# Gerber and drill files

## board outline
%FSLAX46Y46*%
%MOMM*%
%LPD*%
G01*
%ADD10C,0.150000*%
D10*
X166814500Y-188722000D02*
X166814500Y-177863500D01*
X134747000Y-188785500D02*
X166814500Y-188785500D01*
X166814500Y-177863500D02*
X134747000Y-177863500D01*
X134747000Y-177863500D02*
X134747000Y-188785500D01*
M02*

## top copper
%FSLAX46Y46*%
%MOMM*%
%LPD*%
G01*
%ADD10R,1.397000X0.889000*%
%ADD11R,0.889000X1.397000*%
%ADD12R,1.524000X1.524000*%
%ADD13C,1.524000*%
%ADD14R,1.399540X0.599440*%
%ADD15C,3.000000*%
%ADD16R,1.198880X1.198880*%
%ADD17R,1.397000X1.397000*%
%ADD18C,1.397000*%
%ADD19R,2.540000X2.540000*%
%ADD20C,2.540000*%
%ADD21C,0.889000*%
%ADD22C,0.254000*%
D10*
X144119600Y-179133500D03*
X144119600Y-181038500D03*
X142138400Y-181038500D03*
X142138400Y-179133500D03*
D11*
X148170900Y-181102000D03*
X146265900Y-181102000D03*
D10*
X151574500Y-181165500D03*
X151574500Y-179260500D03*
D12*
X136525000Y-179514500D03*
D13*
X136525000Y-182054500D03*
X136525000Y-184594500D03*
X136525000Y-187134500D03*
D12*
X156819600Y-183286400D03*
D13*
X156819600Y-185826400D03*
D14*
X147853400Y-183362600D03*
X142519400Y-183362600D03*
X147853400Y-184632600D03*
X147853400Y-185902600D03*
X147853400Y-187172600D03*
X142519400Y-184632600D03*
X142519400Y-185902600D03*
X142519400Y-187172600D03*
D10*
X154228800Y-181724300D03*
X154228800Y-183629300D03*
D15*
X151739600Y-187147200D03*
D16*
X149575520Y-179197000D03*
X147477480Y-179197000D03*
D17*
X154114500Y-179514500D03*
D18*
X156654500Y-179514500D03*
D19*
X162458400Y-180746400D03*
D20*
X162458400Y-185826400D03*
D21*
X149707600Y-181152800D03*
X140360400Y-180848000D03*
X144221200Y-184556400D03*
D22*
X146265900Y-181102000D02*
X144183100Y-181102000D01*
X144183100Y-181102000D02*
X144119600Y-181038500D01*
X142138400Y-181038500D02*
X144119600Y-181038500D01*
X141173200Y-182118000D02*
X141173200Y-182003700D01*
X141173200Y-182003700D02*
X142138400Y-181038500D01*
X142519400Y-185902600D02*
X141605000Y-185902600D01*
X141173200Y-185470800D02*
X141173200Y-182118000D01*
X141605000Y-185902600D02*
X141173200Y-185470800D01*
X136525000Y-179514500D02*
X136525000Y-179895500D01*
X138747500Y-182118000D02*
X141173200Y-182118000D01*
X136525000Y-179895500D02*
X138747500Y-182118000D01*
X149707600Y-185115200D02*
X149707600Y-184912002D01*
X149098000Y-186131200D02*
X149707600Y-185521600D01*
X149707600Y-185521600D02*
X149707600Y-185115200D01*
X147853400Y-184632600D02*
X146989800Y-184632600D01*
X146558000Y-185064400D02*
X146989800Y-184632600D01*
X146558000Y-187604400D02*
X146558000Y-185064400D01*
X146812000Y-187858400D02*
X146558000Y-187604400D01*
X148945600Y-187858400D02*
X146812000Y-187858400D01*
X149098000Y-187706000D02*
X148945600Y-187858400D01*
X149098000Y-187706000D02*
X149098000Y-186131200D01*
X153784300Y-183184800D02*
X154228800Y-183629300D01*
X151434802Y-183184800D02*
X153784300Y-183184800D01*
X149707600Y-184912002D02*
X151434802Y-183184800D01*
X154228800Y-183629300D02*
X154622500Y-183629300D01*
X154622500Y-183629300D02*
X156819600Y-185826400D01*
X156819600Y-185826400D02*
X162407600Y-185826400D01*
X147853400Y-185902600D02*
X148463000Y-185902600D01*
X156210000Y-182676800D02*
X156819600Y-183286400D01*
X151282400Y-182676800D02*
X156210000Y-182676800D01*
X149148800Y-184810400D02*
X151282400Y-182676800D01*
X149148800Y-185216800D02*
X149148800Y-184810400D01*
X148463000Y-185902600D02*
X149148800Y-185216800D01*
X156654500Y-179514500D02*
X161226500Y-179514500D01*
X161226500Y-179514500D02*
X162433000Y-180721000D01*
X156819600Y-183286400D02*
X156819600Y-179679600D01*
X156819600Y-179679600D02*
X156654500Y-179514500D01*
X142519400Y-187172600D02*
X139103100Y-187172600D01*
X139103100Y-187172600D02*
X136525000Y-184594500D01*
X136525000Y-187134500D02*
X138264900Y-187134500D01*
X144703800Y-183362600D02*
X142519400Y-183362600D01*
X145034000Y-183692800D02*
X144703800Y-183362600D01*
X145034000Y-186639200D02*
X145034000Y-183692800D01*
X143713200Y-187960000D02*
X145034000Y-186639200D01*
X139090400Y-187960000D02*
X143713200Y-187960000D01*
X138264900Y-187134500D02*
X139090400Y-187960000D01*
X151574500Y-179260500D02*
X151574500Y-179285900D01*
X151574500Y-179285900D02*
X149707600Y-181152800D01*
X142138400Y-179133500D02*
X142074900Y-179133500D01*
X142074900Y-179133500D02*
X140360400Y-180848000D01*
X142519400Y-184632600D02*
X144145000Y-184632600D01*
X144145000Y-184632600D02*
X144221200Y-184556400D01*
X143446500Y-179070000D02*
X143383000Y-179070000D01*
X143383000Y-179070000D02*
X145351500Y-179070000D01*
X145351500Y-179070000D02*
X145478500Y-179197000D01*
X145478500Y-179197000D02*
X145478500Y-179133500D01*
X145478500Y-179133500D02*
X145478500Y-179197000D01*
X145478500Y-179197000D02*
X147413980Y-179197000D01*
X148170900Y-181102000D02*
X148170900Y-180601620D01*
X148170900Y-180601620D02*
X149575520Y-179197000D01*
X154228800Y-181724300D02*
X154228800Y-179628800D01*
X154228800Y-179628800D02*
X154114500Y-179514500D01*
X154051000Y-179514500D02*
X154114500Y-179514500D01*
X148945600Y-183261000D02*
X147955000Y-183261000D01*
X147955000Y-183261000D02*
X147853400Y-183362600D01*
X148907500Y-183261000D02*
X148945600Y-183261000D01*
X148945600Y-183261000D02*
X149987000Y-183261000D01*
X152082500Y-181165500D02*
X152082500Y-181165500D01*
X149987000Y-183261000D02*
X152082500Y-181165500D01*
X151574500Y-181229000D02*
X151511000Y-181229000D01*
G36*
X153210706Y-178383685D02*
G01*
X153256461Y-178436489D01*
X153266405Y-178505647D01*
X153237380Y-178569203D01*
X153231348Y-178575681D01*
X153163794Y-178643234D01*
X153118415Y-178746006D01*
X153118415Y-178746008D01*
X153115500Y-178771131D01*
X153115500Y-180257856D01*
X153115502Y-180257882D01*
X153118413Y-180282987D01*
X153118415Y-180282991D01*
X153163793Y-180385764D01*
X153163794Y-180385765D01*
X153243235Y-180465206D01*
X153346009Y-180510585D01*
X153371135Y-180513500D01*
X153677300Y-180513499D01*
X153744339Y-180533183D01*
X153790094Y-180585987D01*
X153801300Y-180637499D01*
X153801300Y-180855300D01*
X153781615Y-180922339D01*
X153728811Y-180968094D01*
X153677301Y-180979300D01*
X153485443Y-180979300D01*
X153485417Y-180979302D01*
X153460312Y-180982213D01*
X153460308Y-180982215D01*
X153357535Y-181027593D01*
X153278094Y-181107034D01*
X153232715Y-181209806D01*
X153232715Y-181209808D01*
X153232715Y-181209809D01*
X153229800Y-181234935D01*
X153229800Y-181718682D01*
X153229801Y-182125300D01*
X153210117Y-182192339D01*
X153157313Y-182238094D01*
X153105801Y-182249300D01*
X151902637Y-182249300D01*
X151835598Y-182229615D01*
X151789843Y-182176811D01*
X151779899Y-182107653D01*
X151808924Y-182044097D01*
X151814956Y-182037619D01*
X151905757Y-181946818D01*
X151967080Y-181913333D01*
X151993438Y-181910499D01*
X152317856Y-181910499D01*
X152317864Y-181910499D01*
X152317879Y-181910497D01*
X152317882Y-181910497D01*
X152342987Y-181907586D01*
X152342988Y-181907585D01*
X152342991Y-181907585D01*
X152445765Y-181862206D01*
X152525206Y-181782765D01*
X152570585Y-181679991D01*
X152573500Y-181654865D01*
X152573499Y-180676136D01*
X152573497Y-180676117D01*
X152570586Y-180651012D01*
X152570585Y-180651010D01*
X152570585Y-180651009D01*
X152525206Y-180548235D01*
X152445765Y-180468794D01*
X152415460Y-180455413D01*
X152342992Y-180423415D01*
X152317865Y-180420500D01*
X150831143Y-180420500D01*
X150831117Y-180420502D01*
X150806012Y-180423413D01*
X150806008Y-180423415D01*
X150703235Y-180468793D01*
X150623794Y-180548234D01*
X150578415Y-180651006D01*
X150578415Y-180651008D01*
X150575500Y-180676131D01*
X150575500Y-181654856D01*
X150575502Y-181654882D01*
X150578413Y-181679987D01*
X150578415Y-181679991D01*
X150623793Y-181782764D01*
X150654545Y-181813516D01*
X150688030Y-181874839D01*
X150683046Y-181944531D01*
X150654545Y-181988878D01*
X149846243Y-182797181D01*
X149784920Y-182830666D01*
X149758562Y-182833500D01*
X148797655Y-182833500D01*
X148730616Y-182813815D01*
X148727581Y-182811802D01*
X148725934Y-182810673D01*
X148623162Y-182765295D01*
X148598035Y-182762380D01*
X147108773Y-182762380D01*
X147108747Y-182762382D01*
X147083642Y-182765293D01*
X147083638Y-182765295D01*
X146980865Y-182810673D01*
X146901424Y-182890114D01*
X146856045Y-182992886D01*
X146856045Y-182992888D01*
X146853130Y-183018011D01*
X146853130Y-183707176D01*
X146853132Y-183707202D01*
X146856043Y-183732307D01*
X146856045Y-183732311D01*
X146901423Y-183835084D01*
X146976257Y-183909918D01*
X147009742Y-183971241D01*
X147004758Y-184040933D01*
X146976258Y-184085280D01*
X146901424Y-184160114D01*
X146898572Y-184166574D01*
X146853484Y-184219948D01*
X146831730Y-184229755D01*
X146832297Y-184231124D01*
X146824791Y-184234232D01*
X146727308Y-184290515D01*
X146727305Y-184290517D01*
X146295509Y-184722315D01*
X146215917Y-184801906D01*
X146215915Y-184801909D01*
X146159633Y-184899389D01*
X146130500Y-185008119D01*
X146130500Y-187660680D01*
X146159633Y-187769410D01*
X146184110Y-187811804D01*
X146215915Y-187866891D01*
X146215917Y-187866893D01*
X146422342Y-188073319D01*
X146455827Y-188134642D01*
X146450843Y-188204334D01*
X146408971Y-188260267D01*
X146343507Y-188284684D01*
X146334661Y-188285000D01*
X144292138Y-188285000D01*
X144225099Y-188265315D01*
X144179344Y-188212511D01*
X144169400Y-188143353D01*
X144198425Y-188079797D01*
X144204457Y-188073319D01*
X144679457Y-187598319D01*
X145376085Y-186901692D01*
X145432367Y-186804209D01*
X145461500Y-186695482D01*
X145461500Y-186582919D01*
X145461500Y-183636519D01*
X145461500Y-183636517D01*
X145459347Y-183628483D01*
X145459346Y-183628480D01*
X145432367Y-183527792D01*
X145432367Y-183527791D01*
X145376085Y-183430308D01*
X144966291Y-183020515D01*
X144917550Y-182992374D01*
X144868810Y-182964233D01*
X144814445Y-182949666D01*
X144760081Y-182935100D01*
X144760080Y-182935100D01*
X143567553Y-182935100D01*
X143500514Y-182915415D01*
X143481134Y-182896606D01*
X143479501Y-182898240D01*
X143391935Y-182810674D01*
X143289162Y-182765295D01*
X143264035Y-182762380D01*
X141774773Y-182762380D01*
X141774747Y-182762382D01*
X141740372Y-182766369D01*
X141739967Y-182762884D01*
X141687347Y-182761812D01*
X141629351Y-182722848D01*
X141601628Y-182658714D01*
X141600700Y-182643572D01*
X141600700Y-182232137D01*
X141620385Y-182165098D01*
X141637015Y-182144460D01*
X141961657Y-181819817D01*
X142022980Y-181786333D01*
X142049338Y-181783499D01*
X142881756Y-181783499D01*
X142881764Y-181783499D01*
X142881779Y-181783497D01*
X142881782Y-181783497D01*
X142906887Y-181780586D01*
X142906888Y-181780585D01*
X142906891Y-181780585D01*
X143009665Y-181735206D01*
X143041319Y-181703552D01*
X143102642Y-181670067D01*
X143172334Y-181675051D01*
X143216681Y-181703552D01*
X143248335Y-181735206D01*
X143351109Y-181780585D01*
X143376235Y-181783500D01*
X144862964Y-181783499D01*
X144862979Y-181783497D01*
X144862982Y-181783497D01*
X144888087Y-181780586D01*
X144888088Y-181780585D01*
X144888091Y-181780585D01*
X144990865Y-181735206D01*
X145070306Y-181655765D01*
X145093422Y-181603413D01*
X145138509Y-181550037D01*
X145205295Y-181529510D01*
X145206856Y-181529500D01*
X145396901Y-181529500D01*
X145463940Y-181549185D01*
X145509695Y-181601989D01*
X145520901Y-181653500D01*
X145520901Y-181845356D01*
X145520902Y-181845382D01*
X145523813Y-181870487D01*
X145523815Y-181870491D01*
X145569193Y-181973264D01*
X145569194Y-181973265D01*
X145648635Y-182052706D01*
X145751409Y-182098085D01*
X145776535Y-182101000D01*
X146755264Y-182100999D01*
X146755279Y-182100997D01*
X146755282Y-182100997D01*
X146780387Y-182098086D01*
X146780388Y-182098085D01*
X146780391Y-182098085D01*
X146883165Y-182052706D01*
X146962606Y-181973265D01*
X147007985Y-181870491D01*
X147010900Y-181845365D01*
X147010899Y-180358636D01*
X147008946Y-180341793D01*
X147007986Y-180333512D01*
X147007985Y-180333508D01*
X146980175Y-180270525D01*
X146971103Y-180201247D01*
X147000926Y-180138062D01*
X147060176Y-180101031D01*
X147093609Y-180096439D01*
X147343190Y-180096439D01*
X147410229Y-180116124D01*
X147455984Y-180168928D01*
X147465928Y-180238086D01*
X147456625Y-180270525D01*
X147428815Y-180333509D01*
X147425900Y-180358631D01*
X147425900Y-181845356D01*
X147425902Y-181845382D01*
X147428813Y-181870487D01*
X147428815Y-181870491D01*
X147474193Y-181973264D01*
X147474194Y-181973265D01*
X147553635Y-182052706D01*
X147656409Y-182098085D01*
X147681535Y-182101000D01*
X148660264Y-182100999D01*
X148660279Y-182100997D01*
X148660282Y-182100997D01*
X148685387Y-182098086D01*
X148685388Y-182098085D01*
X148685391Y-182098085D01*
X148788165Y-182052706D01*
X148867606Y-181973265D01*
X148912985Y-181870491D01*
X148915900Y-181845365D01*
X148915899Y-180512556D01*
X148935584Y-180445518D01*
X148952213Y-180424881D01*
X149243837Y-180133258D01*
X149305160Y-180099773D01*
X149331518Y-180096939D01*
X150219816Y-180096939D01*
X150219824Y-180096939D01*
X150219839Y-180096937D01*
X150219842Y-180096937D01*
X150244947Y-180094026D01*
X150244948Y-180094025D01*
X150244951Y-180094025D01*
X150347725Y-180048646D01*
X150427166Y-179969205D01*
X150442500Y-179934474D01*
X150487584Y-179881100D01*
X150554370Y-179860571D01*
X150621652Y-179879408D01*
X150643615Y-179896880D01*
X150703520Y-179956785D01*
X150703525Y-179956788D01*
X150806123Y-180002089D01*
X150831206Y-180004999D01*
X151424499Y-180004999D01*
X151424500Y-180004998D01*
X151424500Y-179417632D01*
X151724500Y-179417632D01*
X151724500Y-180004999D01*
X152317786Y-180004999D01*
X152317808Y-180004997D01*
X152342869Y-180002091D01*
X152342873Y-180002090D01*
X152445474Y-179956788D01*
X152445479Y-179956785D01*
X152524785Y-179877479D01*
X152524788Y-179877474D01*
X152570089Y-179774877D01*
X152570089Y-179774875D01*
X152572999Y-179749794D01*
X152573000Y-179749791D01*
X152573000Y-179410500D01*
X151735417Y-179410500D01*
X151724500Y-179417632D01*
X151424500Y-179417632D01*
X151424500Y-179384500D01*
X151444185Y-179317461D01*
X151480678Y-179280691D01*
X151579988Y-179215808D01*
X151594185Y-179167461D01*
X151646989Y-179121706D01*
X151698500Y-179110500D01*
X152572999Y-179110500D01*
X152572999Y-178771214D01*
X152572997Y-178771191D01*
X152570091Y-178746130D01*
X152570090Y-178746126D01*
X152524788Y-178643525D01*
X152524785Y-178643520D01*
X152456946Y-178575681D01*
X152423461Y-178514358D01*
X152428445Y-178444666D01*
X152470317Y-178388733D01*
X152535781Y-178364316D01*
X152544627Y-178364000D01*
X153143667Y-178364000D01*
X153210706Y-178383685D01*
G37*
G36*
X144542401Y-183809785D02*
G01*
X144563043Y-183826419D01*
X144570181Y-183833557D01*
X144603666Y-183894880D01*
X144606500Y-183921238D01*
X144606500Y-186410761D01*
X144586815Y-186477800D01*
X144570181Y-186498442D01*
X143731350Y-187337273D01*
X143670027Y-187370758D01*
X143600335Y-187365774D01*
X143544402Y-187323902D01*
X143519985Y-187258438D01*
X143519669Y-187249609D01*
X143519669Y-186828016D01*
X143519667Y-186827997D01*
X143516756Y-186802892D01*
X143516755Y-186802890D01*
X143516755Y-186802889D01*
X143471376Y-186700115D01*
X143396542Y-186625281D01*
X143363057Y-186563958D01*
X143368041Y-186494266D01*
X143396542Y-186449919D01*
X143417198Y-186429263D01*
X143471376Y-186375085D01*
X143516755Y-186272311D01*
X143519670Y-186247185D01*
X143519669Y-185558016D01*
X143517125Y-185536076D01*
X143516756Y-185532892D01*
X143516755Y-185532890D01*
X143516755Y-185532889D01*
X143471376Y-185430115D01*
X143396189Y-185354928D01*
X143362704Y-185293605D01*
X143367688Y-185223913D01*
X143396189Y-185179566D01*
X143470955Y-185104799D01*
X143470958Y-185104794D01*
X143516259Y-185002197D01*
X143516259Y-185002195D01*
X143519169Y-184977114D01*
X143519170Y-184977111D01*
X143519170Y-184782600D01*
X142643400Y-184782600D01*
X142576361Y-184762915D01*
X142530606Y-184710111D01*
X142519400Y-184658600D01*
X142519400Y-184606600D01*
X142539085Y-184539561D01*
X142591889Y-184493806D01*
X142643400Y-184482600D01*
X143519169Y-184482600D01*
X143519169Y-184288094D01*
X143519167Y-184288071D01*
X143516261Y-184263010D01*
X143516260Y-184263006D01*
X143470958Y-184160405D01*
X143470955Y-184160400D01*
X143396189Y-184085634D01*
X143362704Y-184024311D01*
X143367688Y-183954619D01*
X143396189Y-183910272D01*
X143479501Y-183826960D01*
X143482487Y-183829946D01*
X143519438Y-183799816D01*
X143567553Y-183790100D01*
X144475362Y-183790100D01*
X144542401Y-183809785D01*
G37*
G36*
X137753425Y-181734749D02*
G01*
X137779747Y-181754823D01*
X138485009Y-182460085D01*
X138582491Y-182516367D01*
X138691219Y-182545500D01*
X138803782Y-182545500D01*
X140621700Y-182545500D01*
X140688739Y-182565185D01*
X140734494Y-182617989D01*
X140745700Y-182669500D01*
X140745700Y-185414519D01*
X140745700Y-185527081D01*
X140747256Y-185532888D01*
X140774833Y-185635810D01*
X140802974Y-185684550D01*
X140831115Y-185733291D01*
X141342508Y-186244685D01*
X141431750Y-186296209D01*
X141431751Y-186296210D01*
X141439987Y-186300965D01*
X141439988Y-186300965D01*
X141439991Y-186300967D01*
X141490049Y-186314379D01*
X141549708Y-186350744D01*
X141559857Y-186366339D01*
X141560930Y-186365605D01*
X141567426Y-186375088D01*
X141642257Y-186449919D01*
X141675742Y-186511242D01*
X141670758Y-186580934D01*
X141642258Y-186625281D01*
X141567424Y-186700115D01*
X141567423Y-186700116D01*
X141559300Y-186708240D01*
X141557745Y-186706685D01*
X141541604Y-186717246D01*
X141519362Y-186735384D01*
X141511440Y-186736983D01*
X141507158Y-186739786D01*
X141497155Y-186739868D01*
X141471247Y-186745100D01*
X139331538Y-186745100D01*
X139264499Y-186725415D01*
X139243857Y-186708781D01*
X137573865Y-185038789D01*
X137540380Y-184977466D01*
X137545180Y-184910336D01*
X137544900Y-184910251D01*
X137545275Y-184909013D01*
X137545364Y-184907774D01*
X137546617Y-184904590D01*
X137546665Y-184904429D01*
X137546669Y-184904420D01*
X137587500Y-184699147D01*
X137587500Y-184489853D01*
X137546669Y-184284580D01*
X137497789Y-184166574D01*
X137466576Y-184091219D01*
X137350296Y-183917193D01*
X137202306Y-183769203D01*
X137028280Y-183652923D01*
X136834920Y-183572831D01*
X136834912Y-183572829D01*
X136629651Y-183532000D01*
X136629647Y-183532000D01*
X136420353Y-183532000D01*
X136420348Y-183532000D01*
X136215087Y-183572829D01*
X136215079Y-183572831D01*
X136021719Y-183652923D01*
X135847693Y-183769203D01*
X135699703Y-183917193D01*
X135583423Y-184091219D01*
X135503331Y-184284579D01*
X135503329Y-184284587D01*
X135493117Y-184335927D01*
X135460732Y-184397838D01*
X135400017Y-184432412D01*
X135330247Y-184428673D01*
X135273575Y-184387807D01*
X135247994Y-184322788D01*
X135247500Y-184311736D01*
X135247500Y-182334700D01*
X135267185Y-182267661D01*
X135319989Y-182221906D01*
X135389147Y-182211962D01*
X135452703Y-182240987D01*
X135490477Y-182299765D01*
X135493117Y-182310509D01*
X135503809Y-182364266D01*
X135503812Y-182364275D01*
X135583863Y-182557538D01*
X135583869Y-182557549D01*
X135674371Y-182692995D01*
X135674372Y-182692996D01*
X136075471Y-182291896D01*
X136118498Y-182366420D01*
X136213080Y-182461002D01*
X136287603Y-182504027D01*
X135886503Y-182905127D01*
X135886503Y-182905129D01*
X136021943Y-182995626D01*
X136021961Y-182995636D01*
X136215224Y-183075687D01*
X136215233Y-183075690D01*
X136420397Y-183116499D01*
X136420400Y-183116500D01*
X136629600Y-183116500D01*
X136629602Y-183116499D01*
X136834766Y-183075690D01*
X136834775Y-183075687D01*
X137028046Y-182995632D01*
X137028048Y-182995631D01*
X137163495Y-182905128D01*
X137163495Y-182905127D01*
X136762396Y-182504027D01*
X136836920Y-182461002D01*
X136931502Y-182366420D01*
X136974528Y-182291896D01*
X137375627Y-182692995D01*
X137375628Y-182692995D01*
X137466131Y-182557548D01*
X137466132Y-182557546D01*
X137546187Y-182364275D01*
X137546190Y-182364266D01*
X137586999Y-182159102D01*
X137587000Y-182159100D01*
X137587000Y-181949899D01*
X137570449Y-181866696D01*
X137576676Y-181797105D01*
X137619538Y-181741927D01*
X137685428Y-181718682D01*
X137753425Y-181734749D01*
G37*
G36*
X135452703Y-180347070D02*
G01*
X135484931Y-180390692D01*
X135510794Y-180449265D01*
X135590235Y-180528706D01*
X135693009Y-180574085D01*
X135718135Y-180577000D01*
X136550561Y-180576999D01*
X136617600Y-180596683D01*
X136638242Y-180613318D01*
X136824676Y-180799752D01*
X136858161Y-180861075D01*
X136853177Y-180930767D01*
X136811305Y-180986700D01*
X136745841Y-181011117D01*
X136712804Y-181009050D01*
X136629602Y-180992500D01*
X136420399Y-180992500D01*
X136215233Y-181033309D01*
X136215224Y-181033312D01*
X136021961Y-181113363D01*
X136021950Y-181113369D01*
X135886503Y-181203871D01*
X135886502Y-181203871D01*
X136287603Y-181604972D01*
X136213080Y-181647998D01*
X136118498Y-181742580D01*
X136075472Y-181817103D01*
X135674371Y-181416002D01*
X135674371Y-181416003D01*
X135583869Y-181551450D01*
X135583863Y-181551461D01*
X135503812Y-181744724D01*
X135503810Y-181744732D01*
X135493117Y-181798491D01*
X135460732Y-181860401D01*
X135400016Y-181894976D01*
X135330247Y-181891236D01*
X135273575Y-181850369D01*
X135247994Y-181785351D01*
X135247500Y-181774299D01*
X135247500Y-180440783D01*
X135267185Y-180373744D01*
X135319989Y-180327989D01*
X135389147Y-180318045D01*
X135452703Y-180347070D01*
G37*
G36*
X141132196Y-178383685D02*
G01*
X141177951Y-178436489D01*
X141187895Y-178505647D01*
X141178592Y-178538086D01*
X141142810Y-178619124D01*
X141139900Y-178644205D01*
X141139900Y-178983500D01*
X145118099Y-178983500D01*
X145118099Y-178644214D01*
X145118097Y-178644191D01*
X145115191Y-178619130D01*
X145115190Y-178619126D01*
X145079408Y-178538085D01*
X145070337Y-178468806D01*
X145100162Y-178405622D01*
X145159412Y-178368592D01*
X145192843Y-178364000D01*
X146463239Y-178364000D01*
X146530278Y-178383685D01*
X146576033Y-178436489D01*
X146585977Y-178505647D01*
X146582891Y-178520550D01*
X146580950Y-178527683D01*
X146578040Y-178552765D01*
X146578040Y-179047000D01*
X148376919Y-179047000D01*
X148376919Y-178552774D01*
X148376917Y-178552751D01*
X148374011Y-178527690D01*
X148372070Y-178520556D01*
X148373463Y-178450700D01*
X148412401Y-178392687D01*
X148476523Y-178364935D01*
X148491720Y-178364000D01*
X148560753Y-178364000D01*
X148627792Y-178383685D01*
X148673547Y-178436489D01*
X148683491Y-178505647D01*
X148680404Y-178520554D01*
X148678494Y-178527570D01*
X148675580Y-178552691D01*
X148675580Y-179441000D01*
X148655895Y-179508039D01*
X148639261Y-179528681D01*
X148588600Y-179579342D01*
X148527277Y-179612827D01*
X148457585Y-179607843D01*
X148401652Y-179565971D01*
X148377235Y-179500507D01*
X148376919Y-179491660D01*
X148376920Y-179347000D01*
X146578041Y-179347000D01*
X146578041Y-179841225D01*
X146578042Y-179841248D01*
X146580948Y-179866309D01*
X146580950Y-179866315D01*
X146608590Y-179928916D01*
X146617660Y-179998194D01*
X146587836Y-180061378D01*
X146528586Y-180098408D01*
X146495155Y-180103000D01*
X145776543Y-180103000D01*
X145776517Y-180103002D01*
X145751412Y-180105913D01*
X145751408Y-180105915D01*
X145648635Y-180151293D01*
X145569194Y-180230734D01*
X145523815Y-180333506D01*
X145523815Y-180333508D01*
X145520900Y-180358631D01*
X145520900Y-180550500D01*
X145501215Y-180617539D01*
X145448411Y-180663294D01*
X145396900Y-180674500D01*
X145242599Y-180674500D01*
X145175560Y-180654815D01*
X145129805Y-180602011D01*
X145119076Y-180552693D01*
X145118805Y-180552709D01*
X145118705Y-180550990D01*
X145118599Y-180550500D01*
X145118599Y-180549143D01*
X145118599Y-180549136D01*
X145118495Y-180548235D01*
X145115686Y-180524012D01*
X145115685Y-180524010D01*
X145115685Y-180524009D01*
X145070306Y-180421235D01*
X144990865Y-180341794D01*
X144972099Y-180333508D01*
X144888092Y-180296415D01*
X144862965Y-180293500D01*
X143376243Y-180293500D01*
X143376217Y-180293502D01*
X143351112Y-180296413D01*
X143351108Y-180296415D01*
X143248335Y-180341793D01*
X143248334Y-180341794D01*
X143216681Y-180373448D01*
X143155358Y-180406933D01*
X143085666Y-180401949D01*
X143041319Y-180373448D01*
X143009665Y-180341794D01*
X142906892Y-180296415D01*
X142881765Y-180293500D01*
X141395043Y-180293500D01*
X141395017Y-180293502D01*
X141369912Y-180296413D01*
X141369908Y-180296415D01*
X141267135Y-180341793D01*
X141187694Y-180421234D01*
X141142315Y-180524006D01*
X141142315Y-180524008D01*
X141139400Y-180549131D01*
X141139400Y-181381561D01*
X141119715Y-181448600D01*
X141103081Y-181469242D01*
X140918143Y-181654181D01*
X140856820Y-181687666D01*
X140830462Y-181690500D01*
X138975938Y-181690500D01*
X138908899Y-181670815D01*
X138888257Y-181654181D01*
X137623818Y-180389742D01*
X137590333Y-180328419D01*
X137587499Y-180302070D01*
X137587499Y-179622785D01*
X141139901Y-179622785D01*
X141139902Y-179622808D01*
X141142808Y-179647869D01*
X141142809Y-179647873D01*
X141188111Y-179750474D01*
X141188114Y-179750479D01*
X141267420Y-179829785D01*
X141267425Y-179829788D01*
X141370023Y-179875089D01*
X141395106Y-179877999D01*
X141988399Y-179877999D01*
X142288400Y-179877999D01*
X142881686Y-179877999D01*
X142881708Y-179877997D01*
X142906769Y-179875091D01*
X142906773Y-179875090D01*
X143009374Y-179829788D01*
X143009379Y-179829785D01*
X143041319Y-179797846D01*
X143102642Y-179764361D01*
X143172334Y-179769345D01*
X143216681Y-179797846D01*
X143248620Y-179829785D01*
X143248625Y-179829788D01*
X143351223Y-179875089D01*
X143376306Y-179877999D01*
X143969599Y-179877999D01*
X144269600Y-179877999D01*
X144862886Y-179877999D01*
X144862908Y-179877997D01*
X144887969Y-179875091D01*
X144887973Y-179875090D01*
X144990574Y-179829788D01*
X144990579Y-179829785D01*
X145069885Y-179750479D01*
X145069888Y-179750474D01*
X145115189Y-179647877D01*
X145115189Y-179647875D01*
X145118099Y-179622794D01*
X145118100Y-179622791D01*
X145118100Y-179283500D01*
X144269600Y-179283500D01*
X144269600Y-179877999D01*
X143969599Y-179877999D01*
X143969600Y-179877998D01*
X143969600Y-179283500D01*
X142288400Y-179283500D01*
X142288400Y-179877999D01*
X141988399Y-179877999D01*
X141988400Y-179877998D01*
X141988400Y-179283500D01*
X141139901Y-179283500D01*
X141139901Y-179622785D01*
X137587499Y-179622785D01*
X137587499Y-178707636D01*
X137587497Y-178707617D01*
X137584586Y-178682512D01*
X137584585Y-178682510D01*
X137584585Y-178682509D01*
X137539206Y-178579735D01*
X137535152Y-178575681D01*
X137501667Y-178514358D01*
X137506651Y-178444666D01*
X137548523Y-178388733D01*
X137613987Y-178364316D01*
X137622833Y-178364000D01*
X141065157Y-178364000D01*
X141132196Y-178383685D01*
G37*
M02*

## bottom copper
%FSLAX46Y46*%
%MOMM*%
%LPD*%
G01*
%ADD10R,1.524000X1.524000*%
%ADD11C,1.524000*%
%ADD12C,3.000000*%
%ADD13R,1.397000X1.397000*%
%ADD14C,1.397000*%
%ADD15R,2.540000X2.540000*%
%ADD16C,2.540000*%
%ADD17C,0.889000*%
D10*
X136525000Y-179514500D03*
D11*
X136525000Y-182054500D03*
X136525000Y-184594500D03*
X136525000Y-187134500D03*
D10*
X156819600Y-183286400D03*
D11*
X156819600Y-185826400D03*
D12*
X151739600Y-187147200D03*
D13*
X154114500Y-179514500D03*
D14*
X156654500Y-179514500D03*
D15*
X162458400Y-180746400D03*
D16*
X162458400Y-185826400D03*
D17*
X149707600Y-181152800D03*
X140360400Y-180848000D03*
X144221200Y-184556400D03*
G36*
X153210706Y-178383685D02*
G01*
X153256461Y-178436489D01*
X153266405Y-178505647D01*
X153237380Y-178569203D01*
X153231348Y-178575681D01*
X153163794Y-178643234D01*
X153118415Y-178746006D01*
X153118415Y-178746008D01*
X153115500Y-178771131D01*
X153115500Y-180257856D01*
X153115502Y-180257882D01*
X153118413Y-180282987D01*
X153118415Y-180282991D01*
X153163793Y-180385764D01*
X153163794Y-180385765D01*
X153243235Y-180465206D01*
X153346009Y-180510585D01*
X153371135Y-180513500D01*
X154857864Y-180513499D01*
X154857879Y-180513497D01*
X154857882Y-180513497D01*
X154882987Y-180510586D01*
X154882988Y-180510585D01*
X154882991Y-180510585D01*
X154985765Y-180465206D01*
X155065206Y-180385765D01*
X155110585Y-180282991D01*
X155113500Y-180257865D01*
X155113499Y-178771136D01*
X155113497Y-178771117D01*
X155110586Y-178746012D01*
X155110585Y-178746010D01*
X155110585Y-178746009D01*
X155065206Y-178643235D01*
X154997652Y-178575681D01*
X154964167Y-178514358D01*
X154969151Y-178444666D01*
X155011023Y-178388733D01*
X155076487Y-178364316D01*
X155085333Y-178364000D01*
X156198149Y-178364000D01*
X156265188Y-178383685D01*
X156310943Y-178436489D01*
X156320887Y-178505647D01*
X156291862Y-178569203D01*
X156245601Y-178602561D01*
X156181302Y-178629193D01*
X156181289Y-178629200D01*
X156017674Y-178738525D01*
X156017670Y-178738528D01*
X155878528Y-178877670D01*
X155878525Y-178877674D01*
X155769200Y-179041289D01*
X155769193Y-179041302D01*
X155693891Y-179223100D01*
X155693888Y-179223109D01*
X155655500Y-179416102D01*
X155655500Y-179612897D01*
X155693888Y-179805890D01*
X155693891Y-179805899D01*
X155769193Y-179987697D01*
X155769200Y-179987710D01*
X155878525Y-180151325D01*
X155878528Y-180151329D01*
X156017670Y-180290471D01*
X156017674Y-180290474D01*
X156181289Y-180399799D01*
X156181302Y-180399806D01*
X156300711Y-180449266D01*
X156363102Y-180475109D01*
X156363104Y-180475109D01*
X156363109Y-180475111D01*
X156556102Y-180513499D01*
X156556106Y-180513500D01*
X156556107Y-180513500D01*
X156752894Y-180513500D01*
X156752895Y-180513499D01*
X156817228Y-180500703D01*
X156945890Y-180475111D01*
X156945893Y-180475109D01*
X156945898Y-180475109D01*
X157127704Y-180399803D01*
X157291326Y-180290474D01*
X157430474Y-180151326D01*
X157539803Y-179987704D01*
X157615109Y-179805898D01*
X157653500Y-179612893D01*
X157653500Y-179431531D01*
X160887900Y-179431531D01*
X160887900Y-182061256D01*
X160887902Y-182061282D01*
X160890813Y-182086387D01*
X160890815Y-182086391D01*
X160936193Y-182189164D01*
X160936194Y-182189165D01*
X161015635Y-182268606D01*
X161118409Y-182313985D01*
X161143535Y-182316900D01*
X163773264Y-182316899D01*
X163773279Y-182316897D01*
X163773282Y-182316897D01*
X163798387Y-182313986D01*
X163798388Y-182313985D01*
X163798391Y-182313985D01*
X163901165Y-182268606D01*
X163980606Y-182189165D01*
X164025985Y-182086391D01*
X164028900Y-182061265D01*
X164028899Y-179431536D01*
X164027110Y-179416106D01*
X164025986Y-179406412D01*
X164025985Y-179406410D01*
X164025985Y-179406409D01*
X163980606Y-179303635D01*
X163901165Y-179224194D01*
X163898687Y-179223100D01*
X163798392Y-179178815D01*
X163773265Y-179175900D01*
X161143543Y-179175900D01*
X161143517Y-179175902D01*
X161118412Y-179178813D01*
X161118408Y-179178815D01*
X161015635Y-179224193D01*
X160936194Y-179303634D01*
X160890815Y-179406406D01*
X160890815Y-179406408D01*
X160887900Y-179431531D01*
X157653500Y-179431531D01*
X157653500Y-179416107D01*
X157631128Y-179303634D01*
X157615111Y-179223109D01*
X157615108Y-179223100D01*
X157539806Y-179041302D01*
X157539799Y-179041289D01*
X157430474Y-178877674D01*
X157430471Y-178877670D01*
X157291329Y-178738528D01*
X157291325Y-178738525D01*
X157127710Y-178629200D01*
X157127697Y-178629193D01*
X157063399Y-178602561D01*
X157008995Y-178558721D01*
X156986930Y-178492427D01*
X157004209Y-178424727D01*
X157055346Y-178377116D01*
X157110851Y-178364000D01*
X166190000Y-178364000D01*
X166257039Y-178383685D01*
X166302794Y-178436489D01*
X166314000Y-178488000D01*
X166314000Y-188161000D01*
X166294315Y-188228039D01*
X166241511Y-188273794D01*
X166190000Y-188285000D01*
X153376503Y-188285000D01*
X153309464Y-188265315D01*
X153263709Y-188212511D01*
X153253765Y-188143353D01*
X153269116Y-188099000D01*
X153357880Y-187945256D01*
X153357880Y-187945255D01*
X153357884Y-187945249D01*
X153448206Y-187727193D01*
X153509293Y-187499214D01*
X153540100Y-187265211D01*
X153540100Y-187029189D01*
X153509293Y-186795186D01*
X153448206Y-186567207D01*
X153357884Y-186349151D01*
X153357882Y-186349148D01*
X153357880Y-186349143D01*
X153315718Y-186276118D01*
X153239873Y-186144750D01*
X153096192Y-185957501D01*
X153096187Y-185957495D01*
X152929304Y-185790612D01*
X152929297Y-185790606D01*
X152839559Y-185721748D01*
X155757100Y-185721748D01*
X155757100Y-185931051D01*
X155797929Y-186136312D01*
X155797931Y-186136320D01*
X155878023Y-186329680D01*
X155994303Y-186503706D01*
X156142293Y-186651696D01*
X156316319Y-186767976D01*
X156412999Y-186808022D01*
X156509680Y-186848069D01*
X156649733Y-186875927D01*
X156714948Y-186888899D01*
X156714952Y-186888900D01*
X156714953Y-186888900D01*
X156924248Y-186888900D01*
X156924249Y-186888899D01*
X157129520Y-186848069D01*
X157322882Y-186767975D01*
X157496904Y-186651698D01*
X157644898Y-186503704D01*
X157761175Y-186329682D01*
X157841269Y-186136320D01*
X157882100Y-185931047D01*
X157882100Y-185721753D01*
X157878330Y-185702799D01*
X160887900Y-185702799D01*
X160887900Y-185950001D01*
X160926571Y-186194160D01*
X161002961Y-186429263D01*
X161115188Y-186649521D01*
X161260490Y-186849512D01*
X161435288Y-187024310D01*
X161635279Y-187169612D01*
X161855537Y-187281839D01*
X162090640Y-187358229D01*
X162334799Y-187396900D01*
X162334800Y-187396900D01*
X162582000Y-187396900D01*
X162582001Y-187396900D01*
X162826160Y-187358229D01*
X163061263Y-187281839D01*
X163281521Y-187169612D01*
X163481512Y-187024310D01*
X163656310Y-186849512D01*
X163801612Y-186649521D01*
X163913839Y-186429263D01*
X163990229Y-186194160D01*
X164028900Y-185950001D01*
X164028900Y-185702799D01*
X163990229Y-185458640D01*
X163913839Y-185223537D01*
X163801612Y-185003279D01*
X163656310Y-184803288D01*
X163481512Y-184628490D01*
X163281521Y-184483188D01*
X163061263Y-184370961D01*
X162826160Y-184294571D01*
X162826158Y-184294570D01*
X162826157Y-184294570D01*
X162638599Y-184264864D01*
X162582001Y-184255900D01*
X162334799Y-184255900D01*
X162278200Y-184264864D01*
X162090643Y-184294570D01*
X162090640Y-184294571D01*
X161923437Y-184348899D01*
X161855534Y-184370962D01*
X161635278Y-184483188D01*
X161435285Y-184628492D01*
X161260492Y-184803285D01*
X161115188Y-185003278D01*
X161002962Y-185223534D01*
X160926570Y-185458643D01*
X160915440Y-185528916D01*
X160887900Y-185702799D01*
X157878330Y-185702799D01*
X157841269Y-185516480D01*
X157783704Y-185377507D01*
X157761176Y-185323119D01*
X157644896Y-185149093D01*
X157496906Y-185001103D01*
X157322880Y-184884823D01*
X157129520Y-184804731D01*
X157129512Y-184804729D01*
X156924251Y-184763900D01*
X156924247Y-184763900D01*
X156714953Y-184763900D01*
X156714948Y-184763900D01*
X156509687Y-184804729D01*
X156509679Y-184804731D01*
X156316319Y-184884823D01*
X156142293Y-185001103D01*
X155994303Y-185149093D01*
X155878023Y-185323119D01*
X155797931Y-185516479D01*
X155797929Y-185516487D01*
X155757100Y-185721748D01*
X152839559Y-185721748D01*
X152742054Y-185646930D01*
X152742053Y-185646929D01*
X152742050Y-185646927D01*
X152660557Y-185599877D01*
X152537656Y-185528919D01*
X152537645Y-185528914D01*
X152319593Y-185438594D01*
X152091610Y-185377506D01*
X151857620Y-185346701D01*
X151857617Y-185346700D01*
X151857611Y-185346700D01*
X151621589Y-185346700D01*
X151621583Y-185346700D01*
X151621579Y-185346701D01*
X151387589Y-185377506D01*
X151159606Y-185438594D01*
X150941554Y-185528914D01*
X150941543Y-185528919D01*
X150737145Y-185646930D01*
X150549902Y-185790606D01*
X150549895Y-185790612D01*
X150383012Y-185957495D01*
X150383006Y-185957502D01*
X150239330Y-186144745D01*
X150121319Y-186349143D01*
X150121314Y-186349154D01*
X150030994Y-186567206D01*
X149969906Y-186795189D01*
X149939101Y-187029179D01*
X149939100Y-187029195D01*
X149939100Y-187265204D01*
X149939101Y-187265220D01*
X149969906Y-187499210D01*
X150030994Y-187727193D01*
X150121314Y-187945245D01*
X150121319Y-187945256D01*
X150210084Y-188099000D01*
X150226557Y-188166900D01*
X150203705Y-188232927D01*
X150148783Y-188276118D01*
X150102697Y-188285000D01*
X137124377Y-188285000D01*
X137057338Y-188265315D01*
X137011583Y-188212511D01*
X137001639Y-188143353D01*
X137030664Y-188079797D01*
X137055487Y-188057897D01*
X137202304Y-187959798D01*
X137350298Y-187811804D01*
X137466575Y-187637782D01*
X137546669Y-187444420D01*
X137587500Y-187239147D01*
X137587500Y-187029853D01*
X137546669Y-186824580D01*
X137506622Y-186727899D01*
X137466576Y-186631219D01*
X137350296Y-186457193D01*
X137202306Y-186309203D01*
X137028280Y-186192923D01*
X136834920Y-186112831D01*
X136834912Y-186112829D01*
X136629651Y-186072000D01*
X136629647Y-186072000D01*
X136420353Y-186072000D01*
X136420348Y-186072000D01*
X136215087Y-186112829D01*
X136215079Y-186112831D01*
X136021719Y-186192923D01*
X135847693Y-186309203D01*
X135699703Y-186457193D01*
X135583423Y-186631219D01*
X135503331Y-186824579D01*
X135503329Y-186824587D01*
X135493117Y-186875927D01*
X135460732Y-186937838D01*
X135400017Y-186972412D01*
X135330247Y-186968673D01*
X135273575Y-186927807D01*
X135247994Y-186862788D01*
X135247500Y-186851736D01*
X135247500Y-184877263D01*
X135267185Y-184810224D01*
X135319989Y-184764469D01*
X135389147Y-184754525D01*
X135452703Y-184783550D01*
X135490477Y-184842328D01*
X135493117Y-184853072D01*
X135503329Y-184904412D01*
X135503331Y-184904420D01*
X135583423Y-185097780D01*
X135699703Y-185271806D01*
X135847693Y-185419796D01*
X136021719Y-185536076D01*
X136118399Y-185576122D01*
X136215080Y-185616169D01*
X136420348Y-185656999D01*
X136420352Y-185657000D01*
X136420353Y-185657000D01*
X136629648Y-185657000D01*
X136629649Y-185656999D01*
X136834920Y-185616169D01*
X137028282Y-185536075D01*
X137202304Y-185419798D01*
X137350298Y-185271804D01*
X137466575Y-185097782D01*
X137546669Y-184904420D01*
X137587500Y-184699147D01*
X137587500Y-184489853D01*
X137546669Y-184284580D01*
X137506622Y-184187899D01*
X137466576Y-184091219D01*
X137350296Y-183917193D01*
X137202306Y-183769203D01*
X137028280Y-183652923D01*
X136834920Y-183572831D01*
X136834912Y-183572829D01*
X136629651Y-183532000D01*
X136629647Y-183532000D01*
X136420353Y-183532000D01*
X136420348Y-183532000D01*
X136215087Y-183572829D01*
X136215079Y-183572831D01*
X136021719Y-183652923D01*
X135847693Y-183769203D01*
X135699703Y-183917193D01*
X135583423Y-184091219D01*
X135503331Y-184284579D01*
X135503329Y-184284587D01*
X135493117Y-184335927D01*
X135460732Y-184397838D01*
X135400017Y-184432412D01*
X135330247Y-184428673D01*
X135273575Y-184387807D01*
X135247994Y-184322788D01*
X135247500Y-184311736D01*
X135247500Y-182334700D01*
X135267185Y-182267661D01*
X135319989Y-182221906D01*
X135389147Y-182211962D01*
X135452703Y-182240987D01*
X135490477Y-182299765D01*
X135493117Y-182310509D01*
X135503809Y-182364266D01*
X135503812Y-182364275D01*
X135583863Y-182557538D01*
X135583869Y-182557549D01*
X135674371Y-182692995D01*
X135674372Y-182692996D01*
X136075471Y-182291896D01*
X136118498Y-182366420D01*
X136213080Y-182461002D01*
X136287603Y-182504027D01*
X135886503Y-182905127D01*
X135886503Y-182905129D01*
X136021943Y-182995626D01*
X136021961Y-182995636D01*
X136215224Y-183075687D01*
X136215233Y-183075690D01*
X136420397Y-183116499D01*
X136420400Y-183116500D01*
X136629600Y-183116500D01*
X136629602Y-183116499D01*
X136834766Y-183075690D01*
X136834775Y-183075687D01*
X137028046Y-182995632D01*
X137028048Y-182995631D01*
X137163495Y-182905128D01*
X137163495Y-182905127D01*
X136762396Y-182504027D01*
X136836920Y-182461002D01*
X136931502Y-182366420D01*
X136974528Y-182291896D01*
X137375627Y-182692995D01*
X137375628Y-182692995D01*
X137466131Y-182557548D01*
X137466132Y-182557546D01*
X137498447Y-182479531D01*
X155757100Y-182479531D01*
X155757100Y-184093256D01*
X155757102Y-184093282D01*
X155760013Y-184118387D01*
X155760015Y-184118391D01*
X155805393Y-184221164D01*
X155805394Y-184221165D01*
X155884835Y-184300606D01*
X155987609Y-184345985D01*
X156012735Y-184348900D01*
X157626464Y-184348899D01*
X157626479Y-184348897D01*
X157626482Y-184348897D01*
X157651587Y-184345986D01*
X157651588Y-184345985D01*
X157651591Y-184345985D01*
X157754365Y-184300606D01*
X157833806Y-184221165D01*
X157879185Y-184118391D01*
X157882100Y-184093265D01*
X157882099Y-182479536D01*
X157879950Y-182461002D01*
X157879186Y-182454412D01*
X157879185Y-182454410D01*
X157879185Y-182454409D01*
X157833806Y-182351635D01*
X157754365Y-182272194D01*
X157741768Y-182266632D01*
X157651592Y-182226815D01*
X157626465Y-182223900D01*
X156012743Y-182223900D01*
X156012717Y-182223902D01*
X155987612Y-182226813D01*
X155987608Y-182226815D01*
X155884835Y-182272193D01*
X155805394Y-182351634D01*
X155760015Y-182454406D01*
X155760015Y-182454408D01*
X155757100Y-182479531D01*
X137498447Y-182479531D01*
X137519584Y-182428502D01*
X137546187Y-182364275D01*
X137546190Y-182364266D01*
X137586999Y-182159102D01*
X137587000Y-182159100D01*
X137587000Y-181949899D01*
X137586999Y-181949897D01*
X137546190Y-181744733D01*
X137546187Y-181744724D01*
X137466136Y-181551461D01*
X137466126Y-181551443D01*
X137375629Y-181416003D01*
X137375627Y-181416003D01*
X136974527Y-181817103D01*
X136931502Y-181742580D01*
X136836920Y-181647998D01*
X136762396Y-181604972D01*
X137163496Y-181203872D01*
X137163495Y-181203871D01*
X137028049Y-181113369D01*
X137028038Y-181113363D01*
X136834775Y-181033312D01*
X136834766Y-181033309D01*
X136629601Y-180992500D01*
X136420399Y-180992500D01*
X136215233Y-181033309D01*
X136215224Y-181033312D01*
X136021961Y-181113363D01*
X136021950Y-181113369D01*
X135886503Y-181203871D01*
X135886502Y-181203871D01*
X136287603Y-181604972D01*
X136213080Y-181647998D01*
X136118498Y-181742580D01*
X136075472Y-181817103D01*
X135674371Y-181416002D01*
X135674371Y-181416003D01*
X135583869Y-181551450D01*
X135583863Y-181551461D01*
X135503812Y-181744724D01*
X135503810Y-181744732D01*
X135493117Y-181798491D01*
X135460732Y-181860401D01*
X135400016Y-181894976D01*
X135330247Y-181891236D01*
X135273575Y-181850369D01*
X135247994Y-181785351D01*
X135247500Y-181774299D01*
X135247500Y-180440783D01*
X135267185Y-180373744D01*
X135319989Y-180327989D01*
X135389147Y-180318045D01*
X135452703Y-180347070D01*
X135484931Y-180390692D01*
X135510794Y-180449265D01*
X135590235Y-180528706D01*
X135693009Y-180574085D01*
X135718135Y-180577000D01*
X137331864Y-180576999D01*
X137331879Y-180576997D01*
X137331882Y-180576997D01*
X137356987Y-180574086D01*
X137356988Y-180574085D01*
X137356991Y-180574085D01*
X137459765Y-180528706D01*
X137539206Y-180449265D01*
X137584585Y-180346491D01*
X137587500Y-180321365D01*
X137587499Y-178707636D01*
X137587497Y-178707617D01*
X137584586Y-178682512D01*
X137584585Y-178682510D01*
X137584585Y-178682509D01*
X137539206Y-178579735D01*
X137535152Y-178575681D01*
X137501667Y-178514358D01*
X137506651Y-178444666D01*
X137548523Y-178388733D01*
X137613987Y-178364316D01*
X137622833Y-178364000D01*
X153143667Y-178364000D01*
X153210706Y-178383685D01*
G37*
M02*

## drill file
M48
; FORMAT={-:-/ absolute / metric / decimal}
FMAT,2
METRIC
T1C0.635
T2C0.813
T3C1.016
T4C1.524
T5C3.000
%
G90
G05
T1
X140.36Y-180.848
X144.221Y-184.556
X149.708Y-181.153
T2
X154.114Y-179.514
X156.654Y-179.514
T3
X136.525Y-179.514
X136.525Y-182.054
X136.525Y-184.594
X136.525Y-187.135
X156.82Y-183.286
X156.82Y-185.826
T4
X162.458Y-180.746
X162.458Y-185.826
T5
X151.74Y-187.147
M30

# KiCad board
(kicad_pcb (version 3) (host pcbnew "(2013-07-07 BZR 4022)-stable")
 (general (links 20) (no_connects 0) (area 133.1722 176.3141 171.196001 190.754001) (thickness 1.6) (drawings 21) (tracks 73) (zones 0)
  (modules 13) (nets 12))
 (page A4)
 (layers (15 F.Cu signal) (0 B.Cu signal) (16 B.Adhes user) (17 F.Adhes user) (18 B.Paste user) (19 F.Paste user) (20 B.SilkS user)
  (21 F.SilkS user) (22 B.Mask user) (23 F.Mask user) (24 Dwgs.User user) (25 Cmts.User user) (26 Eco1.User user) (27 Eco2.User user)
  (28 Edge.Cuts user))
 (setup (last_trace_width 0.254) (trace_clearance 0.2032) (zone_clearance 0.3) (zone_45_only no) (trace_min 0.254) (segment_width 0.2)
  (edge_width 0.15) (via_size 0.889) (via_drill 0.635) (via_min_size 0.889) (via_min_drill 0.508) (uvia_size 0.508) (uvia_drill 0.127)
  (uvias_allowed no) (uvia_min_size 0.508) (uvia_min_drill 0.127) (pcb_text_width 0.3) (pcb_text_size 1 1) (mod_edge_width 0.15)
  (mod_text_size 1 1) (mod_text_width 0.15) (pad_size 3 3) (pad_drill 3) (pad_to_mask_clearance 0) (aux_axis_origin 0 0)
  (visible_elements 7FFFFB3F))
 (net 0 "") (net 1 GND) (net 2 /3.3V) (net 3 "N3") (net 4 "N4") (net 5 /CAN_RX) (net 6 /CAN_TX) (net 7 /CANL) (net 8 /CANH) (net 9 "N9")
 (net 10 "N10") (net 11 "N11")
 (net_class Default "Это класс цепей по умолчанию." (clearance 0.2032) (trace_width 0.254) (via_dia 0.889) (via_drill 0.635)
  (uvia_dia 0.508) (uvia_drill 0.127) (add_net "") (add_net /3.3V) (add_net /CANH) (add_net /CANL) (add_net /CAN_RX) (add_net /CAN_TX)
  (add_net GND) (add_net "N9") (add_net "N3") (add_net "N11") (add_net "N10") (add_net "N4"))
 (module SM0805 (layer F.Cu) (at 144.1196 180.086 270)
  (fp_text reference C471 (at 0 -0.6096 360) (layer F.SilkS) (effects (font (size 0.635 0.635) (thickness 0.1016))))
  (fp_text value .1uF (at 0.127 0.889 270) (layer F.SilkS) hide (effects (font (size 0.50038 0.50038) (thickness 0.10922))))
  (pad 1 smd rect (at -0.9525 0 270) (size 0.889 1.397) (layers F.Cu F.Paste F.Mask) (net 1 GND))
  (pad 2 smd rect (at 0.9525 0 270) (size 0.889 1.397) (layers F.Cu F.Paste F.Mask) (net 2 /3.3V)))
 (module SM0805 (layer F.Cu) (at 142.1384 180.086 90)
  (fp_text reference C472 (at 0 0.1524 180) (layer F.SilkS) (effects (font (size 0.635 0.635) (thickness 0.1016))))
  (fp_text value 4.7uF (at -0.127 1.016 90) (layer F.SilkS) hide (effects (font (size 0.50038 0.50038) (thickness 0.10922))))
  (pad 1 smd rect (at -0.9525 0 90) (size 0.889 1.397) (layers F.Cu F.Paste F.Mask) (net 2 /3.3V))
  (pad 2 smd rect (at 0.9525 0 90) (size 0.889 1.397) (layers F.Cu F.Paste F.Mask) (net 1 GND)))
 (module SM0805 (layer F.Cu) (at 147.2184 181.102 180)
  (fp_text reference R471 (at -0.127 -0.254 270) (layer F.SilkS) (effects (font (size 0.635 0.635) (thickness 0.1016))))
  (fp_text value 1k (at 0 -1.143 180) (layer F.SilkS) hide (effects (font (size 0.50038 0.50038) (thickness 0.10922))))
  (pad 1 smd rect (at -0.9525 0 180) (size 0.889 1.397) (layers F.Cu F.Paste F.Mask) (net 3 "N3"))
  (pad 2 smd rect (at 0.9525 0 180) (size 0.889 1.397) (layers F.Cu F.Paste F.Mask) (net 2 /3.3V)))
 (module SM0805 (layer F.Cu) (at 151.5745 180.213 90)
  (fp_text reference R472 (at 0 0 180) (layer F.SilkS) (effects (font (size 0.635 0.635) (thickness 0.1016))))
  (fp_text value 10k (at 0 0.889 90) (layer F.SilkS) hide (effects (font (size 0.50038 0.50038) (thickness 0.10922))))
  (pad 1 smd rect (at -0.9525 0 90) (size 0.889 1.397) (layers F.Cu F.Paste F.Mask) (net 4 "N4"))
  (pad 2 smd rect (at 0.9525 0 90) (size 0.889 1.397) (layers F.Cu F.Paste F.Mask) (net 1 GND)))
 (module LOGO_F (layer B.Cu) (at 146.4564 182.7784)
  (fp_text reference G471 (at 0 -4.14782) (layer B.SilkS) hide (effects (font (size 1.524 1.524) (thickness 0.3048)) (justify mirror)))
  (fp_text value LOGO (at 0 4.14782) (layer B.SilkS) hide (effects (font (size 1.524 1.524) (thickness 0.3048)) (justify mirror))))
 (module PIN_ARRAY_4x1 (layer F.Cu) (at 136.525 183.3245 270)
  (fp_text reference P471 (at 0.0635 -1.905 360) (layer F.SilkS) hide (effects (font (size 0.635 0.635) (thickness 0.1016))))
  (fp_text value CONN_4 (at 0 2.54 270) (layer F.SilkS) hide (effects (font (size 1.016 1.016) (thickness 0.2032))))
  (pad 1 thru_hole rect (at -3.81 0 270) (size 1.524 1.524) (drill 1.016) (layers *.Cu *.Mask F.SilkS) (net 2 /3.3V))
  (pad 2 thru_hole circle (at -1.27 0 270) (size 1.524 1.524) (drill 1.016) (layers *.Cu *.Mask F.SilkS) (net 1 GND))
  (pad 3 thru_hole circle (at 1.27 0 270) (size 1.524 1.524) (drill 1.016) (layers *.Cu *.Mask F.SilkS) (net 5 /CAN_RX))
  (pad 4 thru_hole circle (at 3.81 0 270) (size 1.524 1.524) (drill 1.016) (layers *.Cu *.Mask F.SilkS) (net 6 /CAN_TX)))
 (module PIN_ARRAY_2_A (layer F.Cu) (at 156.8196 184.5564 270)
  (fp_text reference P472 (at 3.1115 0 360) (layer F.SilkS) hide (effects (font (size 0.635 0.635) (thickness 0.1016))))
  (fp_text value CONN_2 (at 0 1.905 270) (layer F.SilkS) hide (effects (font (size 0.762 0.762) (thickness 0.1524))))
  (pad 1 thru_hole rect (at -1.27 0 270) (size 1.524 1.524) (drill 1.016) (layers *.Cu *.Mask F.SilkS) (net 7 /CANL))
  (pad 2 thru_hole circle (at 1.27 0 270) (size 1.524 1.524) (drill 1.016) (layers *.Cu *.Mask F.SilkS) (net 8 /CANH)))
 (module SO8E (layer F.Cu) (at 145.1864 185.2676 270)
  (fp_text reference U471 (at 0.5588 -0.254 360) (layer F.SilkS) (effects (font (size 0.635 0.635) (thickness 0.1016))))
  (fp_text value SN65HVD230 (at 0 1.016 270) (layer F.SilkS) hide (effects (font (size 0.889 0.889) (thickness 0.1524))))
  (pad 8 smd rect (at -1.905 -2.667 270) (size 0.59944 1.39954) (layers F.Cu F.Paste F.Mask) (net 4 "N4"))
  (pad 1 smd rect (at -1.905 2.667 270) (size 0.59944 1.39954) (layers F.Cu F.Paste F.Mask) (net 6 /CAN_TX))
  (pad 7 smd rect (at -0.635 -2.667 270) (size 0.59944 1.39954) (layers F.Cu F.Paste F.Mask) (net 8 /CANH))
  (pad 6 smd rect (at 0.635 -2.667 270) (size 0.59944 1.39954) (layers F.Cu F.Paste F.Mask) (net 7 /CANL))
  (pad 5 smd rect (at 1.905 -2.667 270) (size 0.59944 1.39954) (layers F.Cu F.Paste F.Mask) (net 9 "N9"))
  (pad 2 smd rect (at -0.635 2.667 270) (size 0.59944 1.39954) (layers F.Cu F.Paste F.Mask) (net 1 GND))
  (pad 3 smd rect (at 0.635 2.667 270) (size 0.59944 1.39954) (layers F.Cu F.Paste F.Mask) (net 2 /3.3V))
  (pad 4 smd rect (at 1.905 2.667 270) (size 0.59944 1.39954) (layers F.Cu F.Paste F.Mask) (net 5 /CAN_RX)))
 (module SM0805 (layer F.Cu) (at 154.2288 182.6768 270)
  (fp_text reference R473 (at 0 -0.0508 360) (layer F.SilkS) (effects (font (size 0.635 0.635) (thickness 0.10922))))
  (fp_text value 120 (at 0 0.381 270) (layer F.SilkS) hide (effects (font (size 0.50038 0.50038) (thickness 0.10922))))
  (pad 1 smd rect (at -0.9525 0 270) (size 0.889 1.397) (layers F.Cu F.Paste F.Mask) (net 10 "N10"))
  (pad 2 smd rect (at 0.9525 0 270) (size 0.889 1.397) (layers F.Cu F.Paste F.Mask) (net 8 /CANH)))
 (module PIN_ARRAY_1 (layer F.Cu) (at 151.7396 187.1472)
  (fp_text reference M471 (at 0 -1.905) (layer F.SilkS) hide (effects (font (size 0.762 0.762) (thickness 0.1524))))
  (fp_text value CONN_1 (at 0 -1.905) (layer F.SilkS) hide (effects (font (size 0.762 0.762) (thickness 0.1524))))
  (pad 1 thru_hole circle (at 0 0) (size 3 3) (drill 3) (layers *.Cu *.Mask F.SilkS) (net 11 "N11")))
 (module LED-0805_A (layer F.Cu) (at 148.5265 179.197 180)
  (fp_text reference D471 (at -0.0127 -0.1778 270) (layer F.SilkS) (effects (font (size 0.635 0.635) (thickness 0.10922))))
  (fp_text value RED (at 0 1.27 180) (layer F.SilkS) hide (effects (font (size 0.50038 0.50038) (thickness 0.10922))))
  (pad 1 smd rect (at -1.04902 0 180) (size 1.19888 1.19888) (layers F.Cu F.Paste F.Mask) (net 3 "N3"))
  (pad 2 smd rect (at 1.04902 0 180) (size 1.19888 1.19888) (layers F.Cu F.Paste F.Mask) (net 1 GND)))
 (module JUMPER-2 (layer F.Cu) (at 155.3845 179.5145)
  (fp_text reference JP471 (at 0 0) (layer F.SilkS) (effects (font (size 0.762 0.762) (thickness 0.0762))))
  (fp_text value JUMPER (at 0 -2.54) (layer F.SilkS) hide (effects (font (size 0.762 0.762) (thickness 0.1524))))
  (pad 1 thru_hole rect (at -1.27 0) (size 1.397 1.397) (drill 0.8128) (layers *.Cu *.Mask F.SilkS) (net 10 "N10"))
  (pad 2 thru_hole circle (at 1.27 0) (size 1.397 1.397) (drill 0.8128) (layers *.Cu *.Mask F.SilkS) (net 7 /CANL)))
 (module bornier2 (layer F.Cu) (at 162.4584 183.2864 270)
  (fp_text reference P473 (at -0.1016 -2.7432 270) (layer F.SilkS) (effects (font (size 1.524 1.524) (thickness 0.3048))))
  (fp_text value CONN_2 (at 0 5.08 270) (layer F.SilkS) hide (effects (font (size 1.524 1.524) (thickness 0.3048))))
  (pad 1 thru_hole rect (at -2.54 0 270) (size 2.54 2.54) (drill 1.524) (layers *.Cu *.Mask F.SilkS) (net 7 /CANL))
  (pad 2 thru_hole circle (at 2.54 0 270) (size 2.54 2.54) (drill 1.524) (layers *.Cu *.Mask F.SilkS) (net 8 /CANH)))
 (gr_line (start 166.8145 188.722) (end 166.8145 177.8635) (angle 90) (layer Edge.Cuts) (width 0.15))
 (gr_line (start 134.747 188.7855) (end 166.8145 188.7855) (angle 90) (layer Edge.Cuts) (width 0.15))
 (gr_line (start 166.8145 177.8635) (end 134.747 177.8635) (angle 90) (layer Edge.Cuts) (width 0.15))
 (gr_line (start 134.747 177.8635) (end 134.747 188.7855) (angle 90) (layer Edge.Cuts) (width 0.15))
 (segment (start 146.2659 181.102) (end 144.1831 181.102) (width 0.254) (layer F.Cu) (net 2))
 (segment (start 144.1831 181.102) (end 144.1196 181.0385) (width 0.254) (layer F.Cu) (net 2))
 (segment (start 142.1384 181.0385) (end 144.1196 181.0385) (width 0.254) (layer F.Cu) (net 2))
 (segment (start 141.1732 182.118) (end 141.1732 182.0037) (width 0.254) (layer F.Cu) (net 2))
 (segment (start 141.1732 182.0037) (end 142.1384 181.0385) (width 0.254) (layer F.Cu) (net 2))
 (segment (start 142.5194 185.9026) (end 141.605 185.9026) (width 0.254) (layer F.Cu) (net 2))
 (segment (start 141.1732 185.4708) (end 141.1732 182.118) (width 0.254) (layer F.Cu) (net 2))
 (segment (start 141.605 185.9026) (end 141.1732 185.4708) (width 0.254) (layer F.Cu) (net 2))
 (segment (start 136.525 179.5145) (end 136.525 179.8955) (width 0.254) (layer F.Cu) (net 2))
 (segment (start 138.7475 182.118) (end 141.1732 182.118) (width 0.254) (layer F.Cu) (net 2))
 (segment (start 136.525 179.8955) (end 138.7475 182.118) (width 0.254) (layer F.Cu) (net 2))
 (segment (start 149.7076 185.1152) (end 149.7076 184.912002) (width 0.254) (layer F.Cu) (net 8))
 (segment (start 149.098 186.1312) (end 149.7076 185.5216) (width 0.254) (layer F.Cu) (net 8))
 (segment (start 149.7076 185.5216) (end 149.7076 185.1152) (width 0.254) (layer F.Cu) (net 8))
 (segment (start 147.8534 184.6326) (end 146.9898 184.6326) (width 0.254) (layer F.Cu) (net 8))
 (segment (start 146.558 185.0644) (end 146.9898 184.6326) (width 0.254) (layer F.Cu) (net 8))
 (segment (start 146.558 187.6044) (end 146.558 185.0644) (width 0.254) (layer F.Cu) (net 8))
 (segment (start 146.812 187.8584) (end 146.558 187.6044) (width 0.254) (layer F.Cu) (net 8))
 (segment (start 148.9456 187.8584) (end 146.812 187.8584) (width 0.254) (layer F.Cu) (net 8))
 (segment (start 149.098 187.706) (end 148.9456 187.8584) (width 0.254) (layer F.Cu) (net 8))
 (segment (start 149.098 187.706) (end 149.098 186.1312) (width 0.254) (layer F.Cu) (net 8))
 (segment (start 153.7843 183.1848) (end 154.2288 183.6293) (width 0.254) (layer F.Cu) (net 8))
 (segment (start 151.434802 183.1848) (end 153.7843 183.1848) (width 0.254) (layer F.Cu) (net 8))
 (segment (start 149.7076 184.912002) (end 151.434802 183.1848) (width 0.254) (layer F.Cu) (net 8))
 (segment (start 154.2288 183.6293) (end 154.6225 183.6293) (width 0.254) (layer F.Cu) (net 8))
 (segment (start 154.6225 183.6293) (end 156.8196 185.8264) (width 0.254) (layer F.Cu) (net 8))
 (segment (start 156.8196 185.8264) (end 162.4076 185.8264) (width 0.254) (layer F.Cu) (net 8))
 (segment (start 147.8534 185.9026) (end 148.463 185.9026) (width 0.254) (layer F.Cu) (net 7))
 (segment (start 156.21 182.6768) (end 156.8196 183.2864) (width 0.254) (layer F.Cu) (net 7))
 (segment (start 151.2824 182.6768) (end 156.21 182.6768) (width 0.254) (layer F.Cu) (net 7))
 (segment (start 149.1488 184.8104) (end 151.2824 182.6768) (width 0.254) (layer F.Cu) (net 7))
 (segment (start 149.1488 185.2168) (end 149.1488 184.8104) (width 0.254) (layer F.Cu) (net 7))
 (segment (start 148.463 185.9026) (end 149.1488 185.2168) (width 0.254) (layer F.Cu) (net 7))
 (segment (start 156.6545 179.5145) (end 161.2265 179.5145) (width 0.254) (layer F.Cu) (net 7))
 (segment (start 161.2265 179.5145) (end 162.433 180.721) (width 0.254) (layer F.Cu) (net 7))
 (segment (start 156.8196 183.2864) (end 156.8196 179.6796) (width 0.254) (layer F.Cu) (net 7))
 (segment (start 156.8196 179.6796) (end 156.6545 179.5145) (width 0.254) (layer F.Cu) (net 7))
 (segment (start 142.5194 187.1726) (end 139.1031 187.1726) (width 0.254) (layer F.Cu) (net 5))
 (segment (start 139.1031 187.1726) (end 136.525 184.5945) (width 0.254) (layer F.Cu) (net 5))
 (segment (start 136.525 187.1345) (end 138.2649 187.1345) (width 0.254) (layer F.Cu) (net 6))
 (segment (start 144.7038 183.3626) (end 142.5194 183.3626) (width 0.254) (layer F.Cu) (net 6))
 (segment (start 145.034 183.6928) (end 144.7038 183.3626) (width 0.254) (layer F.Cu) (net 6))
 (segment (start 145.034 186.6392) (end 145.034 183.6928) (width 0.254) (layer F.Cu) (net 6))
 (segment (start 143.7132 187.96) (end 145.034 186.6392) (width 0.254) (layer F.Cu) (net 6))
 (segment (start 139.0904 187.96) (end 143.7132 187.96) (width 0.254) (layer F.Cu) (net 6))
 (segment (start 138.2649 187.1345) (end 139.0904 187.96) (width 0.254) (layer F.Cu) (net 6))
 (segment (start 151.5745 179.2605) (end 151.5745 179.2859) (width 0.254) (layer F.Cu) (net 1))
 (via (at 149.7076 181.1528) (size 0.889) (layers F.Cu B.Cu) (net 1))
 (segment (start 151.5745 179.2859) (end 149.7076 181.1528) (width 0.254) (layer F.Cu) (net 1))
 (segment (start 142.1384 179.1335) (end 142.0749 179.1335) (width 0.254) (layer F.Cu) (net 1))
 (via (at 140.3604 180.848) (size 0.889) (layers F.Cu B.Cu) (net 1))
 (segment (start 142.0749 179.1335) (end 140.3604 180.848) (width 0.254) (layer F.Cu) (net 1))
 (segment (start 142.5194 184.6326) (end 144.145 184.6326) (width 0.254) (layer F.Cu) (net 1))
 (via (at 144.2212 184.5564) (size 0.889) (layers F.Cu B.Cu) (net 1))
 (segment (start 144.145 184.6326) (end 144.2212 184.5564) (width 0.254) (layer F.Cu) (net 1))
 (segment (start 143.4465 179.07) (end 143.383 179.07) (width 0.254) (layer F.Cu) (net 1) (status 80000))
 (segment (start 143.383 179.07) (end 145.3515 179.07) (width 0.254) (layer F.Cu) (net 1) (status 80000))
 (segment (start 145.3515 179.07) (end 145.4785 179.197) (width 0.254) (layer F.Cu) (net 1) (status 80000))
 (segment (start 145.4785 179.197) (end 145.4785 179.1335) (width 0.254) (layer F.Cu) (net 1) (status 80000))
 (segment (start 145.4785 179.1335) (end 145.4785 179.197) (width 0.254) (layer F.Cu) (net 1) (status 80000))
 (segment (start 145.4785 179.197) (end 147.41398 179.197) (width 0.254) (layer F.Cu) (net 1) (status 80000))
 (segment (start 148.1709 181.102) (end 148.1709 180.60162) (width 0.254) (layer F.Cu) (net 3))
 (segment (start 148.1709 180.60162) (end 149.57552 179.197) (width 0.254) (layer F.Cu) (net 3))
 (segment (start 154.2288 181.7243) (end 154.2288 179.6288) (width 0.254) (layer F.Cu) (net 10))
 (segment (start 154.2288 179.6288) (end 154.1145 179.5145) (width 0.254) (layer F.Cu) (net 10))
 (segment (start 154.051 179.5145) (end 154.1145 179.5145) (width 0.254) (layer F.Cu) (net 10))
 (segment (start 148.9456 183.261) (end 147.955 183.261) (width 0.254) (layer F.Cu) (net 4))
 (segment (start 147.955 183.261) (end 147.8534 183.3626) (width 0.254) (layer F.Cu) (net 4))
 (segment (start 148.9075 183.261) (end 148.9456 183.261) (width 0.254) (layer F.Cu) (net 4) (status 10))
 (segment (start 148.9456 183.261) (end 149.987 183.261) (width 0.254) (layer F.Cu) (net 4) (status 10))
 (segment (start 152.0825 181.1655) (end 152.0825 181.1655) (width 0.254) (layer F.Cu) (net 4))
 (segment (start 149.987 183.261) (end 152.0825 181.1655) (width 0.254) (layer F.Cu) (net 4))
 (segment (start 151.5745 181.229) (end 151.511 181.229) (width 0.254) (layer F.Cu) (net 4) (status 80000))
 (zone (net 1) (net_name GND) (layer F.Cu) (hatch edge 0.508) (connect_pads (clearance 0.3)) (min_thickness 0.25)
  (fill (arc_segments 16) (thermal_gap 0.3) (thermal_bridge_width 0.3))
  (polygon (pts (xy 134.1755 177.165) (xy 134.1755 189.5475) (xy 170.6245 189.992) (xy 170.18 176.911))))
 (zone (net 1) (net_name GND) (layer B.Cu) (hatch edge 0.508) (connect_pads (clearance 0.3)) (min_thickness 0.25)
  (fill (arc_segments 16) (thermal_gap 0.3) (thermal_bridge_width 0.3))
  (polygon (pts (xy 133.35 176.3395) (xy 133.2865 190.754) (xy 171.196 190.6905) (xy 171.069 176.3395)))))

